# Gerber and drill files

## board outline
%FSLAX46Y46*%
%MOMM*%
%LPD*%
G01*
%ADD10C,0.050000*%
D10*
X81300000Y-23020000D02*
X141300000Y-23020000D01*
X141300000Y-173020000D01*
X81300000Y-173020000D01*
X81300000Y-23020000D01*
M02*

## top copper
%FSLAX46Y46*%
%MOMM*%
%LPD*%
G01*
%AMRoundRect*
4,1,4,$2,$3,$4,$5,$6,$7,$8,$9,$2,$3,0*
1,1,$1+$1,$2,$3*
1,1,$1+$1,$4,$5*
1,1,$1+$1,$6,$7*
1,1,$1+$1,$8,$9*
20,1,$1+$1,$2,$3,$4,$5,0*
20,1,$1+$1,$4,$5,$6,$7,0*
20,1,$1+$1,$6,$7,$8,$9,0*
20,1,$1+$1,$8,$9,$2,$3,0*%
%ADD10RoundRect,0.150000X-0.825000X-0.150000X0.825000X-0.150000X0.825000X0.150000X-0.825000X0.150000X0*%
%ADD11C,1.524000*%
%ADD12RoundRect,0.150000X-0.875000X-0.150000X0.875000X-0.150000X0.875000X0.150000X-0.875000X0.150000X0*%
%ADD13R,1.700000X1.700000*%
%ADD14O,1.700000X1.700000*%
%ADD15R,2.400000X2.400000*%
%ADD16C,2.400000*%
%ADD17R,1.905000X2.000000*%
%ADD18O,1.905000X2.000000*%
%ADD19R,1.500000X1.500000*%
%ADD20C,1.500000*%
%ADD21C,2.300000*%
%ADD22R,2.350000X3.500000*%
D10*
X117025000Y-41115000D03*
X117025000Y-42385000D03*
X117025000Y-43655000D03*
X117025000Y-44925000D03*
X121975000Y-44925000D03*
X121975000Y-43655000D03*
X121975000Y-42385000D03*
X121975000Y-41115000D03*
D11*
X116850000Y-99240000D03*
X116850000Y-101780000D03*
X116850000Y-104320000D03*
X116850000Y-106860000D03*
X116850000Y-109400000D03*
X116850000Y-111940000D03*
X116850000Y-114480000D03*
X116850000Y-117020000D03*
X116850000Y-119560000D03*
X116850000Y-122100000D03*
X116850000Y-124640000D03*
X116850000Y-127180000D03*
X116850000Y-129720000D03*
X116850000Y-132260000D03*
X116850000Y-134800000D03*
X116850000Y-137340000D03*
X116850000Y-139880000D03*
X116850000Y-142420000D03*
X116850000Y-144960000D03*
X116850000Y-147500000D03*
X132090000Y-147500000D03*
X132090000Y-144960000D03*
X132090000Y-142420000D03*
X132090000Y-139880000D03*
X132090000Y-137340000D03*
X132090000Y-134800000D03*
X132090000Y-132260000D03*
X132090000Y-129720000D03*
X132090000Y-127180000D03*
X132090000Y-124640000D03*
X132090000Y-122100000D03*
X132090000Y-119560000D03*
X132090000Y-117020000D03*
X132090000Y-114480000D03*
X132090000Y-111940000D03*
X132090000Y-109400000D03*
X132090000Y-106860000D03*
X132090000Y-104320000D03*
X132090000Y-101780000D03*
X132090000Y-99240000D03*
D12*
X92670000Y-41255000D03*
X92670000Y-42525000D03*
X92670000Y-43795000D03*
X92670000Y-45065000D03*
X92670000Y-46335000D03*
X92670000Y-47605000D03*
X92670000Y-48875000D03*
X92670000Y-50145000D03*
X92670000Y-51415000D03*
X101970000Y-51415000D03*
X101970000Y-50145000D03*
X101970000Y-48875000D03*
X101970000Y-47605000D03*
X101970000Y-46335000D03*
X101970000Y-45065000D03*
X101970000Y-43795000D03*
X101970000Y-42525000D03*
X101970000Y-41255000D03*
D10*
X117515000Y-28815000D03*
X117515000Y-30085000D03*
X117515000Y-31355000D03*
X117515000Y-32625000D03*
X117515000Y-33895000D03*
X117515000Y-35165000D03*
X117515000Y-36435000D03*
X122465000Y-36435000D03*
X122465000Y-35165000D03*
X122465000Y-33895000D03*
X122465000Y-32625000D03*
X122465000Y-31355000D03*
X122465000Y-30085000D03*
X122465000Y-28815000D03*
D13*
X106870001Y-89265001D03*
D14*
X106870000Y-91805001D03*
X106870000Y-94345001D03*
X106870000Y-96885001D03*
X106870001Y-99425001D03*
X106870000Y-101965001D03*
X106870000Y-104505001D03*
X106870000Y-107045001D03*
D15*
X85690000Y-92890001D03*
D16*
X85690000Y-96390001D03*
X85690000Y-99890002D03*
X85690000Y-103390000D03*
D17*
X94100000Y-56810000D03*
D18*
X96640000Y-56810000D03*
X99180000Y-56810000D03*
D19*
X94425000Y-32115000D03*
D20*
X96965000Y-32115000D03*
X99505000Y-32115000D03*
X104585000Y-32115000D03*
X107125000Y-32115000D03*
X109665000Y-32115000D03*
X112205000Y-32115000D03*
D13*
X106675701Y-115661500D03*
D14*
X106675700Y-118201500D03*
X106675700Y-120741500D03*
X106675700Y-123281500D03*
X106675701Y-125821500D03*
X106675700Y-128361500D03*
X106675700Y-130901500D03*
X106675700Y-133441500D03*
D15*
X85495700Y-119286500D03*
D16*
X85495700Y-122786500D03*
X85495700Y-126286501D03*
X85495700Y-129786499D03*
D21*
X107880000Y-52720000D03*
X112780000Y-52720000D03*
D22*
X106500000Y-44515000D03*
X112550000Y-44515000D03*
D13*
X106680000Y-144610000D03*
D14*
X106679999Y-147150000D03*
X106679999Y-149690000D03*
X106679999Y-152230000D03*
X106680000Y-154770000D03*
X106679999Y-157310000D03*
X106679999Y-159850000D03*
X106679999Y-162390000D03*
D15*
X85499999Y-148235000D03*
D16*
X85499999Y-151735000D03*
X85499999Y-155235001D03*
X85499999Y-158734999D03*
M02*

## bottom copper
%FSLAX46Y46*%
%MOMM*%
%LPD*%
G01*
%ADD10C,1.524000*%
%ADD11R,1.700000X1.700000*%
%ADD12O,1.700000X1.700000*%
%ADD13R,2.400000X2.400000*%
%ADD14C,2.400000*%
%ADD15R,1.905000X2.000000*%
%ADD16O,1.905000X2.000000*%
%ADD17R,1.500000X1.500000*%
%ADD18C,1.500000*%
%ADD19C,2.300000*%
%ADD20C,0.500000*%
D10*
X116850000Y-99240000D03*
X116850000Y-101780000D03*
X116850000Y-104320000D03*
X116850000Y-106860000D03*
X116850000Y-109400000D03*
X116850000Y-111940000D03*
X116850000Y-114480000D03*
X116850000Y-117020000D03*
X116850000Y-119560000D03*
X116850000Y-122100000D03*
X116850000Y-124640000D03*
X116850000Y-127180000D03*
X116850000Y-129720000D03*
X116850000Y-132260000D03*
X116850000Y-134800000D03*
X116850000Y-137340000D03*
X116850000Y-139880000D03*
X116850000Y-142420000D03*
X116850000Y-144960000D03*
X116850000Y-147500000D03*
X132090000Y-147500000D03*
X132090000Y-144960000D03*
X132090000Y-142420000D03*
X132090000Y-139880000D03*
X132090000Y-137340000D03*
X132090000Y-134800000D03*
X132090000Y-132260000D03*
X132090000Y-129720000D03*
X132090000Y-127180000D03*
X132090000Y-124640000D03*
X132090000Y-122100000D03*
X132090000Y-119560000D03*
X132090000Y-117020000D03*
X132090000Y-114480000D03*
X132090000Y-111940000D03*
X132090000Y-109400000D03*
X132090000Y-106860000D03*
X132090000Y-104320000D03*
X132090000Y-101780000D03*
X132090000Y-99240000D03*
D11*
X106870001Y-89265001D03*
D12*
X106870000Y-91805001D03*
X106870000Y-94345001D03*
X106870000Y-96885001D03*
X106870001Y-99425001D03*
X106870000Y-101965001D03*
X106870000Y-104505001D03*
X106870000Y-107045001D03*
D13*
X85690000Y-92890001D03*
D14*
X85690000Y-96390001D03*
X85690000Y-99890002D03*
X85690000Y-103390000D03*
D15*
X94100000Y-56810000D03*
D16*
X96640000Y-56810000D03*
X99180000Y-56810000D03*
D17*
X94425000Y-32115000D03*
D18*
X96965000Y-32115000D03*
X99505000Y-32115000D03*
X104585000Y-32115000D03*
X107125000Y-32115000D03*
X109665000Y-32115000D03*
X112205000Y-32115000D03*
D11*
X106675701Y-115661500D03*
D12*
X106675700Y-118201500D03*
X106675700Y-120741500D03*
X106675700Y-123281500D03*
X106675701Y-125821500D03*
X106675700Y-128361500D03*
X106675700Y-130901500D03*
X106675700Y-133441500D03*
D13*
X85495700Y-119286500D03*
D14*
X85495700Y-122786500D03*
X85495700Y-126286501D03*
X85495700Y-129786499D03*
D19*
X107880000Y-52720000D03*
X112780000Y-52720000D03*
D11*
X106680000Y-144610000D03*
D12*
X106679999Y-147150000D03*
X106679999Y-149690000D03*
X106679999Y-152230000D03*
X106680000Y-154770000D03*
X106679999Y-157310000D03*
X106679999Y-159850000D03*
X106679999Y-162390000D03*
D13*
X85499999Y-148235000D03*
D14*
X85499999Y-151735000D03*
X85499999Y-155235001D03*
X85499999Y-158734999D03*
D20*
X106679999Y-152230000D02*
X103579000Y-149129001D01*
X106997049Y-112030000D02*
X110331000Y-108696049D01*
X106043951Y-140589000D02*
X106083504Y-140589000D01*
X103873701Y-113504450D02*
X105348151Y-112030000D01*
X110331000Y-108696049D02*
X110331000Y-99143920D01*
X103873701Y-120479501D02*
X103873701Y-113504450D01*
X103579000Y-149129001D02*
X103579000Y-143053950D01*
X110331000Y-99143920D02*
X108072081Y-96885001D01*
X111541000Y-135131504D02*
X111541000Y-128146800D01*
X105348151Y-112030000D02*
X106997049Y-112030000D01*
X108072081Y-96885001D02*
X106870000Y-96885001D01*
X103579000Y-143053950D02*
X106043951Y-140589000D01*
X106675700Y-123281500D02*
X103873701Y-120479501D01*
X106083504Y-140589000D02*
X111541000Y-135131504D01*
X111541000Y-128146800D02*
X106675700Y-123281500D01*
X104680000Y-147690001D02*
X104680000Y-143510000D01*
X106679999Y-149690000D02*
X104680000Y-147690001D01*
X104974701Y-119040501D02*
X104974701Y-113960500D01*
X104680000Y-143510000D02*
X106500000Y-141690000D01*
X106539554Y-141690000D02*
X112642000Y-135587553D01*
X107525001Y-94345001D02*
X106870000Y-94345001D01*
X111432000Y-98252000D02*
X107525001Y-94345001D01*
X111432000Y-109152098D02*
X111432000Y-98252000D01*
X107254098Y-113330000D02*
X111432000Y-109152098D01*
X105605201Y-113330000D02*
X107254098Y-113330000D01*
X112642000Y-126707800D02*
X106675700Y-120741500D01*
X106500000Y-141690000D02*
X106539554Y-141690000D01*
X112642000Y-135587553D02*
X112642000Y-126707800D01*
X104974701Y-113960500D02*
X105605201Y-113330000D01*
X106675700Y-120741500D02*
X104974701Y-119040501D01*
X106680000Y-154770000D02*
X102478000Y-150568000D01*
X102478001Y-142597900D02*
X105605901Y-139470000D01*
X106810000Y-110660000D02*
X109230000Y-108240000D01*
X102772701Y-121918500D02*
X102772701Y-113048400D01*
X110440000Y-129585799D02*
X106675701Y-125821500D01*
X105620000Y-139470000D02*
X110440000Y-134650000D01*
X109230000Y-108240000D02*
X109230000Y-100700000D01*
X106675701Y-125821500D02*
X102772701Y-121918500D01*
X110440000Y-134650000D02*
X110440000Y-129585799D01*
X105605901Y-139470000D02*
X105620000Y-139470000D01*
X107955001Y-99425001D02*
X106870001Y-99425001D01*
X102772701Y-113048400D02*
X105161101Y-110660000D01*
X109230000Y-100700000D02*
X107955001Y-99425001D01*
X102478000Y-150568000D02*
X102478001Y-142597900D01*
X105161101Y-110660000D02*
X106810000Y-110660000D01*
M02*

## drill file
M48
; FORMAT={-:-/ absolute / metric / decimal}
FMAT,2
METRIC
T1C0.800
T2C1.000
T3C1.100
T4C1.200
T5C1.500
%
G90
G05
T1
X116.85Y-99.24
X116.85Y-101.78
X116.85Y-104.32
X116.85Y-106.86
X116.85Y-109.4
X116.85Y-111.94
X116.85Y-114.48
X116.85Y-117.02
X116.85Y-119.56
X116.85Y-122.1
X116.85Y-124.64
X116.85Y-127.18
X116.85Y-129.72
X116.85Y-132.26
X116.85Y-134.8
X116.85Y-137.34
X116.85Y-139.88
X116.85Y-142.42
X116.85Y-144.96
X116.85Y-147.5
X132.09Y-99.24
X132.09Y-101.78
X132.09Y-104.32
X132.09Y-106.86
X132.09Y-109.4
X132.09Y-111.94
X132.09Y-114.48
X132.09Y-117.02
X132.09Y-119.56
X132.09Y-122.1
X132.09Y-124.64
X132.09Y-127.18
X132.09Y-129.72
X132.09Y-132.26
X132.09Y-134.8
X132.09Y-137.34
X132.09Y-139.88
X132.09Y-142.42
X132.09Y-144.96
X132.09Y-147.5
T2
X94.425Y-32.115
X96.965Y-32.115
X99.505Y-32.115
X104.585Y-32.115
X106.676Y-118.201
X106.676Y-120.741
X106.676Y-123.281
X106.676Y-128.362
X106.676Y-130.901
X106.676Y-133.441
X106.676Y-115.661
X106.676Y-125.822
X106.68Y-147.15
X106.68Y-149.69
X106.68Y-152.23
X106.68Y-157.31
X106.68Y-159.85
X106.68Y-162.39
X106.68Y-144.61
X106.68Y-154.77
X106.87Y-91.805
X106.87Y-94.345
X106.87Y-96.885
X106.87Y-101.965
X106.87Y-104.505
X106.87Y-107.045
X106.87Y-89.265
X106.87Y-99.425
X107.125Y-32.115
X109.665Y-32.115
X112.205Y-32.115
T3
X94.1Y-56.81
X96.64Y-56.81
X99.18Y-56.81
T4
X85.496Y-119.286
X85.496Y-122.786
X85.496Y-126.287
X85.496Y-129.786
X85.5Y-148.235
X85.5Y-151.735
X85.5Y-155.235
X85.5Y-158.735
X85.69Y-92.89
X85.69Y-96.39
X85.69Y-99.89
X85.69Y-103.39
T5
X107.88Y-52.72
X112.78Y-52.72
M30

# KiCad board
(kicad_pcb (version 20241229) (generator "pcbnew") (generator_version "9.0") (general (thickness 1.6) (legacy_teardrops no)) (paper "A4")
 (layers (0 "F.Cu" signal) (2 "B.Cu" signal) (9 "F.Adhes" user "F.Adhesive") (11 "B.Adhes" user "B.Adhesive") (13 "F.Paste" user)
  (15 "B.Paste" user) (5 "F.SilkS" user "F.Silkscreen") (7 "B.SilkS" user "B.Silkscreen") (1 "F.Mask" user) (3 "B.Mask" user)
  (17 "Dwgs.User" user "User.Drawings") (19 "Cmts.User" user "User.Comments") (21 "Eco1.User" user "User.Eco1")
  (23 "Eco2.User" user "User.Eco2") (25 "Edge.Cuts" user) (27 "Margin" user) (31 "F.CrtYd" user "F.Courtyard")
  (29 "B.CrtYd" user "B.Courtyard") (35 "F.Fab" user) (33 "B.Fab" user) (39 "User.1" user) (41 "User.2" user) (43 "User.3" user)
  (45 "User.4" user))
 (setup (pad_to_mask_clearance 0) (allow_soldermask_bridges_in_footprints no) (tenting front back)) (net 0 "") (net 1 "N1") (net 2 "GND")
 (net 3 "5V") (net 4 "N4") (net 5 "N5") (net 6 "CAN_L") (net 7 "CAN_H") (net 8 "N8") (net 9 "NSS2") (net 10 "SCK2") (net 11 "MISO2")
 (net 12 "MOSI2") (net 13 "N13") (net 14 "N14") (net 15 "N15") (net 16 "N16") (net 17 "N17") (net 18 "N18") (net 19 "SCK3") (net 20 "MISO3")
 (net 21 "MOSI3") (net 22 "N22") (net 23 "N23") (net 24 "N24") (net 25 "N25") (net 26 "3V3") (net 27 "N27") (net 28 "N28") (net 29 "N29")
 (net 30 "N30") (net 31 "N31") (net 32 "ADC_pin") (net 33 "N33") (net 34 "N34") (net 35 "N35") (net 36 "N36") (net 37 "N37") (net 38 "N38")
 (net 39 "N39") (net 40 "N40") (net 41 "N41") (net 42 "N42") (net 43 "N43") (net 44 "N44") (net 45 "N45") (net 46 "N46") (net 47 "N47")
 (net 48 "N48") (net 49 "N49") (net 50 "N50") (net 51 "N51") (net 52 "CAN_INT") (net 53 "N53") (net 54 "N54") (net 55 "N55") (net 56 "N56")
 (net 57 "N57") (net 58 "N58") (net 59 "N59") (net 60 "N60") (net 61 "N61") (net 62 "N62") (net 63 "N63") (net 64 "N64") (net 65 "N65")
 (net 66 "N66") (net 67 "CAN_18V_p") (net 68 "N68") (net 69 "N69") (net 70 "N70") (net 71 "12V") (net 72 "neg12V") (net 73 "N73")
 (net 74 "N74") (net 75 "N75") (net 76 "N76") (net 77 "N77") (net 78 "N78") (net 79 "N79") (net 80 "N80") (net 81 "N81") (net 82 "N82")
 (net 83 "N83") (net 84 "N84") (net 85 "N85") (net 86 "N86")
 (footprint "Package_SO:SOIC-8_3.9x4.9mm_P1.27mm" (layer "F.Cu") (at 119.5 43.02)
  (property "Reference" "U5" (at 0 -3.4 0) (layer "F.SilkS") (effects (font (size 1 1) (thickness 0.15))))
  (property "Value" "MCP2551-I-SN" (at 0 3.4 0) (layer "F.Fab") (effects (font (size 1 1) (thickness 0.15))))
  (pad "1" smd roundrect (at -2.475 -1.905) (size 1.95 0.6) (layers "F.Cu" "F.Mask" "F.Paste") (roundrect_rratio 0.25) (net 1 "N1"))
  (pad "2" smd roundrect (at -2.475 -0.635) (size 1.95 0.6) (layers "F.Cu" "F.Mask" "F.Paste") (roundrect_rratio 0.25) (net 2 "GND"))
  (pad "3" smd roundrect (at -2.475 0.635) (size 1.95 0.6) (layers "F.Cu" "F.Mask" "F.Paste") (roundrect_rratio 0.25) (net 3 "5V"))
  (pad "4" smd roundrect (at -2.475 1.905) (size 1.95 0.6) (layers "F.Cu" "F.Mask" "F.Paste") (roundrect_rratio 0.25) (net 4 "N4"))
  (pad "5" smd roundrect (at 2.475 1.905) (size 1.95 0.6) (layers "F.Cu" "F.Mask" "F.Paste") (roundrect_rratio 0.25) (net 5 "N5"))
  (pad "6" smd roundrect (at 2.475 0.635) (size 1.95 0.6) (layers "F.Cu" "F.Mask" "F.Paste") (roundrect_rratio 0.25) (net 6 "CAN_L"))
  (pad "7" smd roundrect (at 2.475 -0.635) (size 1.95 0.6) (layers "F.Cu" "F.Mask" "F.Paste") (roundrect_rratio 0.25) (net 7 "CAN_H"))
  (pad "8" smd roundrect (at 2.475 -1.905) (size 1.95 0.6) (layers "F.Cu" "F.Mask" "F.Paste") (roundrect_rratio 0.25) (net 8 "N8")))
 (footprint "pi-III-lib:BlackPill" (layer "F.Cu") (at 124.47 120.83)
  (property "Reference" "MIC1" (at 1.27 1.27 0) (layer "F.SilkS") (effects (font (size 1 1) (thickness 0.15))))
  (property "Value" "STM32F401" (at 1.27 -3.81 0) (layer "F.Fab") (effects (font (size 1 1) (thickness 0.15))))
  (pad "1" thru_hole circle (at -7.62 -21.59) (size 1.524 1.524) (drill 0.8) (layers "*.Cu" "*.Mask") (remove_unused_layers no)
   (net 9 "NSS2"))
  (pad "2" thru_hole circle (at -7.62 -19.05) (size 1.524 1.524) (drill 0.8) (layers "*.Cu" "*.Mask") (remove_unused_layers no)
   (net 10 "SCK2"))
  (pad "3" thru_hole circle (at -7.62 -16.51) (size 1.524 1.524) (drill 0.8) (layers "*.Cu" "*.Mask") (remove_unused_layers no)
   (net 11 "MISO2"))
  (pad "4" thru_hole circle (at -7.62 -13.97) (size 1.524 1.524) (drill 0.8) (layers "*.Cu" "*.Mask") (remove_unused_layers no)
   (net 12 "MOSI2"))
  (pad "5" thru_hole circle (at -7.62 -11.43) (size 1.524 1.524) (drill 0.8) (layers "*.Cu" "*.Mask") (remove_unused_layers no)
   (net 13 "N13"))
  (pad "6" thru_hole circle (at -7.62 -8.89) (size 1.524 1.524) (drill 0.8) (layers "*.Cu" "*.Mask") (remove_unused_layers no)
   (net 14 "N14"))
  (pad "7" thru_hole circle (at -7.62 -6.35) (size 1.524 1.524) (drill 0.8) (layers "*.Cu" "*.Mask") (remove_unused_layers no)
   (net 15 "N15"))
  (pad "8" thru_hole circle (at -7.62 -3.81) (size 1.524 1.524) (drill 0.8) (layers "*.Cu" "*.Mask") (remove_unused_layers no)
   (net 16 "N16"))
  (pad "9" thru_hole circle (at -7.62 -1.27) (size 1.524 1.524) (drill 0.8) (layers "*.Cu" "*.Mask") (remove_unused_layers no)
   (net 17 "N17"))
  (pad "10" thru_hole circle (at -7.62 1.27) (size 1.524 1.524) (drill 0.8) (layers "*.Cu" "*.Mask") (remove_unused_layers no)
   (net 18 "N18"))
  (pad "11" thru_hole circle (at -7.62 3.81) (size 1.524 1.524) (drill 0.8) (layers "*.Cu" "*.Mask") (remove_unused_layers no)
   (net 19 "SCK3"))
  (pad "12" thru_hole circle (at -7.62 6.35) (size 1.524 1.524) (drill 0.8) (layers "*.Cu" "*.Mask") (remove_unused_layers no)
   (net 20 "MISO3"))
  (pad "13" thru_hole circle (at -7.62 8.89) (size 1.524 1.524) (drill 0.8) (layers "*.Cu" "*.Mask") (remove_unused_layers no)
   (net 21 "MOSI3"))
  (pad "14" thru_hole circle (at -7.62 11.43) (size 1.524 1.524) (drill 0.8) (layers "*.Cu" "*.Mask") (remove_unused_layers no)
   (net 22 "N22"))
  (pad "15" thru_hole circle (at -7.62 13.97) (size 1.524 1.524) (drill 0.8) (layers "*.Cu" "*.Mask") (remove_unused_layers no)
   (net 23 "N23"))
  (pad "16" thru_hole circle (at -7.62 16.51) (size 1.524 1.524) (drill 0.8) (layers "*.Cu" "*.Mask") (remove_unused_layers no)
   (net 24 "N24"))
  (pad "17" thru_hole circle (at -7.62 19.05) (size 1.524 1.524) (drill 0.8) (layers "*.Cu" "*.Mask") (remove_unused_layers no)
   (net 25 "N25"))
  (pad "18" thru_hole circle (at -7.62 21.59) (size 1.524 1.524) (drill 0.8) (layers "*.Cu" "*.Mask") (remove_unused_layers no) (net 3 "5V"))
  (pad "19" thru_hole circle (at -7.62 24.13) (size 1.524 1.524) (drill 0.8) (layers "*.Cu" "*.Mask") (remove_unused_layers no)
   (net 2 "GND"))
  (pad "20" thru_hole circle (at -7.62 26.67) (size 1.524 1.524) (drill 0.8) (layers "*.Cu" "*.Mask") (remove_unused_layers no)
   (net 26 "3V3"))
  (pad "21" thru_hole circle (at 7.62 26.67) (size 1.524 1.524) (drill 0.8) (layers "*.Cu" "*.Mask") (remove_unused_layers no)
   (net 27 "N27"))
  (pad "22" thru_hole circle (at 7.62 24.13) (size 1.524 1.524) (drill 0.8) (layers "*.Cu" "*.Mask") (remove_unused_layers no)
   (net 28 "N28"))
  (pad "23" thru_hole circle (at 7.62 21.59) (size 1.524 1.524) (drill 0.8) (layers "*.Cu" "*.Mask") (remove_unused_layers no)
   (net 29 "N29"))
  (pad "24" thru_hole circle (at 7.62 19.05) (size 1.524 1.524) (drill 0.8) (layers "*.Cu" "*.Mask") (remove_unused_layers no)
   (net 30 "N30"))
  (pad "25" thru_hole circle (at 7.62 16.51) (size 1.524 1.524) (drill 0.8) (layers "*.Cu" "*.Mask") (remove_unused_layers no)
   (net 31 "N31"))
  (pad "26" thru_hole circle (at 7.62 13.97) (size 1.524 1.524) (drill 0.8) (layers "*.Cu" "*.Mask") (remove_unused_layers no)
   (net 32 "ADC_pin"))
  (pad "27" thru_hole circle (at 7.62 11.43) (size 1.524 1.524) (drill 0.8) (layers "*.Cu" "*.Mask") (remove_unused_layers no)
   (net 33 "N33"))
  (pad "28" thru_hole circle (at 7.62 8.89) (size 1.524 1.524) (drill 0.8) (layers "*.Cu" "*.Mask") (remove_unused_layers no) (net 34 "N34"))
  (pad "29" thru_hole circle (at 7.62 6.35) (size 1.524 1.524) (drill 0.8) (layers "*.Cu" "*.Mask") (remove_unused_layers no) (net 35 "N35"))
  (pad "30" thru_hole circle (at 7.62 3.81) (size 1.524 1.524) (drill 0.8) (layers "*.Cu" "*.Mask") (remove_unused_layers no) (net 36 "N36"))
  (pad "31" thru_hole circle (at 7.62 1.27) (size 1.524 1.524) (drill 0.8) (layers "*.Cu" "*.Mask") (remove_unused_layers no) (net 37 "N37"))
  (pad "32" thru_hole circle (at 7.62 -1.27) (size 1.524 1.524) (drill 0.8) (layers "*.Cu" "*.Mask") (remove_unused_layers no)
   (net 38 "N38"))
  (pad "33" thru_hole circle (at 7.62 -3.81) (size 1.524 1.524) (drill 0.8) (layers "*.Cu" "*.Mask") (remove_unused_layers no)
   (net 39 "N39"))
  (pad "34" thru_hole circle (at 7.62 -6.35) (size 1.524 1.524) (drill 0.8) (layers "*.Cu" "*.Mask") (remove_unused_layers no)
   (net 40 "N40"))
  (pad "35" thru_hole circle (at 7.62 -8.89) (size 1.524 1.524) (drill 0.8) (layers "*.Cu" "*.Mask") (remove_unused_layers no)
   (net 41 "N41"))
  (pad "36" thru_hole circle (at 7.62 -11.43) (size 1.524 1.524) (drill 0.8) (layers "*.Cu" "*.Mask") (remove_unused_layers no)
   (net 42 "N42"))
  (pad "37" thru_hole circle (at 7.62 -13.97) (size 1.524 1.524) (drill 0.8) (layers "*.Cu" "*.Mask") (remove_unused_layers no)
   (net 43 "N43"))
  (pad "38" thru_hole circle (at 7.62 -16.51) (size 1.524 1.524) (drill 0.8) (layers "*.Cu" "*.Mask") (remove_unused_layers no)
   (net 26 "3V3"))
  (pad "39" thru_hole circle (at 7.62 -19.05) (size 1.524 1.524) (drill 0.8) (layers "*.Cu" "*.Mask") (remove_unused_layers no)
   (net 2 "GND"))
  (pad "40" thru_hole circle (at 7.62 -21.59) (size 1.524 1.524) (drill 0.8) (layers "*.Cu" "*.Mask") (remove_unused_layers no) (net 3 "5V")))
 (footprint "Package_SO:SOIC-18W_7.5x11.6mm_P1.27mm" (layer "F.Cu") (at 97.32 46.335)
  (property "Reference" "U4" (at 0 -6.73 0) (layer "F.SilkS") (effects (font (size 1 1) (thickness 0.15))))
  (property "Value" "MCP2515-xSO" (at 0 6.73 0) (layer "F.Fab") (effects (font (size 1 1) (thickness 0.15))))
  (pad "1" smd roundrect (at -4.65 -5.08) (size 2.05 0.6) (layers "F.Cu" "F.Mask" "F.Paste") (roundrect_rratio 0.25) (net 1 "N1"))
  (pad "2" smd roundrect (at -4.65 -3.81) (size 2.05 0.6) (layers "F.Cu" "F.Mask" "F.Paste") (roundrect_rratio 0.25) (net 4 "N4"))
  (pad "3" smd roundrect (at -4.65 -2.54) (size 2.05 0.6) (layers "F.Cu" "F.Mask" "F.Paste") (roundrect_rratio 0.25) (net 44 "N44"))
  (pad "4" smd roundrect (at -4.65 -1.27) (size 2.05 0.6) (layers "F.Cu" "F.Mask" "F.Paste") (roundrect_rratio 0.25) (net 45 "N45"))
  (pad "5" smd roundrect (at -4.65 0) (size 2.05 0.6) (layers "F.Cu" "F.Mask" "F.Paste") (roundrect_rratio 0.25) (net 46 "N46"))
  (pad "6" smd roundrect (at -4.65 1.27) (size 2.05 0.6) (layers "F.Cu" "F.Mask" "F.Paste") (roundrect_rratio 0.25) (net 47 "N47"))
  (pad "7" smd roundrect (at -4.65 2.54) (size 2.05 0.6) (layers "F.Cu" "F.Mask" "F.Paste") (roundrect_rratio 0.25) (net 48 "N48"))
  (pad "8" smd roundrect (at -4.65 3.81) (size 2.05 0.6) (layers "F.Cu" "F.Mask" "F.Paste") (roundrect_rratio 0.25) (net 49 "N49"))
  (pad "9" smd roundrect (at -4.65 5.08) (size 2.05 0.6) (layers "F.Cu" "F.Mask" "F.Paste") (roundrect_rratio 0.25) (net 2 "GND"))
  (pad "10" smd roundrect (at 4.65 5.08) (size 2.05 0.6) (layers "F.Cu" "F.Mask" "F.Paste") (roundrect_rratio 0.25) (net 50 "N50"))
  (pad "11" smd roundrect (at 4.65 3.81) (size 2.05 0.6) (layers "F.Cu" "F.Mask" "F.Paste") (roundrect_rratio 0.25) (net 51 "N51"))
  (pad "12" smd roundrect (at 4.65 2.54) (size 2.05 0.6) (layers "F.Cu" "F.Mask" "F.Paste") (roundrect_rratio 0.25) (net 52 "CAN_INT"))
  (pad "13" smd roundrect (at 4.65 1.27) (size 2.05 0.6) (layers "F.Cu" "F.Mask" "F.Paste") (roundrect_rratio 0.25) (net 10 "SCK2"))
  (pad "14" smd roundrect (at 4.65 0) (size 2.05 0.6) (layers "F.Cu" "F.Mask" "F.Paste") (roundrect_rratio 0.25) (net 12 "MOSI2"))
  (pad "15" smd roundrect (at 4.65 -1.27) (size 2.05 0.6) (layers "F.Cu" "F.Mask" "F.Paste") (roundrect_rratio 0.25) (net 11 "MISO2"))
  (pad "16" smd roundrect (at 4.65 -2.54) (size 2.05 0.6) (layers "F.Cu" "F.Mask" "F.Paste") (roundrect_rratio 0.25) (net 9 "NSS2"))
  (pad "17" smd roundrect (at 4.65 -3.81) (size 2.05 0.6) (layers "F.Cu" "F.Mask" "F.Paste") (roundrect_rratio 0.25) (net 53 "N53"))
  (pad "18" smd roundrect (at 4.65 -5.08) (size 2.05 0.6) (layers "F.Cu" "F.Mask" "F.Paste") (roundrect_rratio 0.25) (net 26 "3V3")))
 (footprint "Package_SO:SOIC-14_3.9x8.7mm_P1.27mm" (layer "F.Cu") (at 119.99 32.625)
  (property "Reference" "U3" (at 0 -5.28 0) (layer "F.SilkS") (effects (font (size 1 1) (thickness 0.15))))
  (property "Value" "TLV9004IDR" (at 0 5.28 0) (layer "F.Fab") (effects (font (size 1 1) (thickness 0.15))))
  (pad "1" smd roundrect (at -2.475 -3.81) (size 1.95 0.6) (layers "F.Cu" "F.Mask" "F.Paste") (roundrect_rratio 0.25) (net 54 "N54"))
  (pad "2" smd roundrect (at -2.475 -2.54) (size 1.95 0.6) (layers "F.Cu" "F.Mask" "F.Paste") (roundrect_rratio 0.25) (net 54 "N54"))
  (pad "3" smd roundrect (at -2.475 -1.27) (size 1.95 0.6) (layers "F.Cu" "F.Mask" "F.Paste") (roundrect_rratio 0.25) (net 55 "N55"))
  (pad "4" smd roundrect (at -2.475 0) (size 1.95 0.6) (layers "F.Cu" "F.Mask" "F.Paste") (roundrect_rratio 0.25) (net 26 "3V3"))
  (pad "5" smd roundrect (at -2.475 1.27) (size 1.95 0.6) (layers "F.Cu" "F.Mask" "F.Paste") (roundrect_rratio 0.25))
  (pad "6" smd roundrect (at -2.475 2.54) (size 1.95 0.6) (layers "F.Cu" "F.Mask" "F.Paste") (roundrect_rratio 0.25))
  (pad "7" smd roundrect (at -2.475 3.81) (size 1.95 0.6) (layers "F.Cu" "F.Mask" "F.Paste") (roundrect_rratio 0.25))
  (pad "8" smd roundrect (at 2.475 3.81) (size 1.95 0.6) (layers "F.Cu" "F.Mask" "F.Paste") (roundrect_rratio 0.25) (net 32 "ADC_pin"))
  (pad "9" smd roundrect (at 2.475 2.54) (size 1.95 0.6) (layers "F.Cu" "F.Mask" "F.Paste") (roundrect_rratio 0.25) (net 32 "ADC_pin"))
  (pad "10" smd roundrect (at 2.475 1.27) (size 1.95 0.6) (layers "F.Cu" "F.Mask" "F.Paste") (roundrect_rratio 0.25) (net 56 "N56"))
  (pad "11" smd roundrect (at 2.475 0) (size 1.95 0.6) (layers "F.Cu" "F.Mask" "F.Paste") (roundrect_rratio 0.25) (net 2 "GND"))
  (pad "12" smd roundrect (at 2.475 -1.27) (size 1.95 0.6) (layers "F.Cu" "F.Mask" "F.Paste") (roundrect_rratio 0.25) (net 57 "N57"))
  (pad "13" smd roundrect (at 2.475 -2.54) (size 1.95 0.6) (layers "F.Cu" "F.Mask" "F.Paste") (roundrect_rratio 0.25) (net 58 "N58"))
  (pad "14" smd roundrect (at 2.475 -3.81) (size 1.95 0.6) (layers "F.Cu" "F.Mask" "F.Paste") (roundrect_rratio 0.25) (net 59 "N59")))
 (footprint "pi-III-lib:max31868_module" (layer "F.Cu") (at 73.31 101.059501 90)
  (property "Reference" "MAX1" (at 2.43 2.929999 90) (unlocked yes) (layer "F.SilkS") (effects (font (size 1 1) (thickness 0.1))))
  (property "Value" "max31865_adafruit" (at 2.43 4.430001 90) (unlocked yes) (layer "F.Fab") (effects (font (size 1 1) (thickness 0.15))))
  (pad "1" thru_hole rect (at 11.7945 33.560001 180) (size 1.7 1.7) (drill 1) (layers "*.Cu" "*.Mask") (remove_unused_layers no)
   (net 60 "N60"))
  (pad "2" thru_hole oval (at 9.2545 33.56 180) (size 1.7 1.7) (drill 1) (layers "*.Cu" "*.Mask") (remove_unused_layers no) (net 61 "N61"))
  (pad "3" thru_hole oval (at 6.7145 33.56 180) (size 1.7 1.7) (drill 1) (layers "*.Cu" "*.Mask") (remove_unused_layers no) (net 21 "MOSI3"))
  (pad "4" thru_hole oval (at 4.1745 33.56 180) (size 1.7 1.7) (drill 1) (layers "*.Cu" "*.Mask") (remove_unused_layers no) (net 20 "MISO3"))
  (pad "5" thru_hole oval (at 1.6345 33.560001 180) (size 1.7 1.7) (drill 1) (layers "*.Cu" "*.Mask") (remove_unused_layers no)
   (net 19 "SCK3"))
  (pad "6" thru_hole oval (at -0.9055 33.56 180) (size 1.7 1.7) (drill 1) (layers "*.Cu" "*.Mask") (remove_unused_layers no) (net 26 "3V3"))
  (pad "7" thru_hole oval (at -3.4455 33.56 180) (size 1.7 1.7) (drill 1) (layers "*.Cu" "*.Mask") (remove_unused_layers no) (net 2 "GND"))
  (pad "8" thru_hole oval (at -5.9855 33.56 180) (size 1.7 1.7) (drill 1) (layers "*.Cu" "*.Mask") (remove_unused_layers no) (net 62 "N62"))
  (pad "9" thru_hole rect (at 8.1695 12.38 270) (size 2.4 2.4) (drill 1.2) (layers "*.Cu" "*.Mask") (remove_unused_layers no) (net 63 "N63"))
  (pad "10" thru_hole circle (at 4.6695 12.38 270) (size 2.4 2.4) (drill 1.2) (layers "*.Cu" "*.Mask") (remove_unused_layers no)
   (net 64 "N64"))
  (pad "11" thru_hole circle (at 1.169499 12.38 270) (size 2.4 2.4) (drill 1.2) (layers "*.Cu" "*.Mask") (remove_unused_layers no)
   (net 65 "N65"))
  (pad "12" thru_hole circle (at -2.330499 12.38 270) (size 2.4 2.4) (drill 1.2) (layers "*.Cu" "*.Mask") (remove_unused_layers no)
   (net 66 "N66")))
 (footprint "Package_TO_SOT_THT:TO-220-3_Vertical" (layer "F.Cu") (at 94.1 56.81)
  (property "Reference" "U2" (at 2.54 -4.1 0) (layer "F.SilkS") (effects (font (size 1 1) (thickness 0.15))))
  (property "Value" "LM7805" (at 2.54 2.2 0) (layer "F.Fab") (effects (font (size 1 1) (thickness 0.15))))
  (pad "1" thru_hole rect (at 0 0) (size 1.905 2) (drill 1.1) (layers "*.Cu" "*.Mask") (remove_unused_layers no) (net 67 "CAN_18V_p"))
  (pad "2" thru_hole oval (at 2.54 0) (size 1.905 2) (drill 1.1) (layers "*.Cu" "*.Mask") (remove_unused_layers no) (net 2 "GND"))
  (pad "3" thru_hole oval (at 5.08 0) (size 1.905 2) (drill 1.1) (layers "*.Cu" "*.Mask") (remove_unused_layers no) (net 3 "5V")))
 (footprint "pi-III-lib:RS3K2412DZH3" (layer "F.Cu") (at 94.425 32.115)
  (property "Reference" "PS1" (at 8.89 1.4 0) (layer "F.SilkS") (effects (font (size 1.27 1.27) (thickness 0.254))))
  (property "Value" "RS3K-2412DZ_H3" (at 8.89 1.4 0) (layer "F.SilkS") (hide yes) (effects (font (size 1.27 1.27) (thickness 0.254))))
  (pad "1" thru_hole rect (at 0 0) (size 1.5 1.5) (drill 1) (layers "*.Cu" "*.Mask") (remove_unused_layers no) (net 2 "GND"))
  (pad "2" thru_hole circle (at 2.54 0) (size 1.5 1.5) (drill 1) (layers "*.Cu" "*.Mask") (remove_unused_layers no) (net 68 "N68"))
  (pad "3" thru_hole circle (at 5.08 0) (size 1.5 1.5) (drill 1) (layers "*.Cu" "*.Mask") (remove_unused_layers no) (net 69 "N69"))
  (pad "5" thru_hole circle (at 10.16 0) (size 1.5 1.5) (drill 1) (layers "*.Cu" "*.Mask") (remove_unused_layers no) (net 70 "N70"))
  (pad "6" thru_hole circle (at 12.7 0) (size 1.5 1.5) (drill 1) (layers "*.Cu" "*.Mask") (remove_unused_layers no) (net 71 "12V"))
  (pad "7" thru_hole circle (at 15.24 0) (size 1.5 1.5) (drill 1) (layers "*.Cu" "*.Mask") (remove_unused_layers no) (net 2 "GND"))
  (pad "8" thru_hole circle (at 17.78 0) (size 1.5 1.5) (drill 1) (layers "*.Cu" "*.Mask") (remove_unused_layers no) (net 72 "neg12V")))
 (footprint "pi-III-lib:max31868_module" (layer "F.Cu") (at 73.1157 127.456 90)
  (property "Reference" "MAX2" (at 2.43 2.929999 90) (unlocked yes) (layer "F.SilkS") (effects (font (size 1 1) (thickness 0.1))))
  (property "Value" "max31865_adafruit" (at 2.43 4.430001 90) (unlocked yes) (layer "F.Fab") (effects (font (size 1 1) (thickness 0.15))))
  (pad "1" thru_hole rect (at 11.7945 33.560001 180) (size 1.7 1.7) (drill 1) (layers "*.Cu" "*.Mask") (remove_unused_layers no)
   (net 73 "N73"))
  (pad "2" thru_hole oval (at 9.2545 33.56 180) (size 1.7 1.7) (drill 1) (layers "*.Cu" "*.Mask") (remove_unused_layers no) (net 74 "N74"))
  (pad "3" thru_hole oval (at 6.7145 33.56 180) (size 1.7 1.7) (drill 1) (layers "*.Cu" "*.Mask") (remove_unused_layers no) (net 21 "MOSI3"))
  (pad "4" thru_hole oval (at 4.1745 33.56 180) (size 1.7 1.7) (drill 1) (layers "*.Cu" "*.Mask") (remove_unused_layers no) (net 20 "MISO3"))
  (pad "5" thru_hole oval (at 1.6345 33.560001 180) (size 1.7 1.7) (drill 1) (layers "*.Cu" "*.Mask") (remove_unused_layers no)
   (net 19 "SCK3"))
  (pad "6" thru_hole oval (at -0.9055 33.56 180) (size 1.7 1.7) (drill 1) (layers "*.Cu" "*.Mask") (remove_unused_layers no) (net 26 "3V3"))
  (pad "7" thru_hole oval (at -3.4455 33.56 180) (size 1.7 1.7) (drill 1) (layers "*.Cu" "*.Mask") (remove_unused_layers no) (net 2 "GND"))
  (pad "8" thru_hole oval (at -5.9855 33.56 180) (size 1.7 1.7) (drill 1) (layers "*.Cu" "*.Mask") (remove_unused_layers no) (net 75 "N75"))
  (pad "9" thru_hole rect (at 8.1695 12.38 270) (size 2.4 2.4) (drill 1.2) (layers "*.Cu" "*.Mask") (remove_unused_layers no) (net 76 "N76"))
  (pad "10" thru_hole circle (at 4.6695 12.38 270) (size 2.4 2.4) (drill 1.2) (layers "*.Cu" "*.Mask") (remove_unused_layers no)
   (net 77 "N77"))
  (pad "11" thru_hole circle (at 1.169499 12.38 270) (size 2.4 2.4) (drill 1.2) (layers "*.Cu" "*.Mask") (remove_unused_layers no)
   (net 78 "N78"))
  (pad "12" thru_hole circle (at -2.330499 12.38 270) (size 2.4 2.4) (drill 1.2) (layers "*.Cu" "*.Mask") (remove_unused_layers no)
   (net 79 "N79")))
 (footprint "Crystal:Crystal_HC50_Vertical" (layer "F.Cu") (at 107.88 52.72)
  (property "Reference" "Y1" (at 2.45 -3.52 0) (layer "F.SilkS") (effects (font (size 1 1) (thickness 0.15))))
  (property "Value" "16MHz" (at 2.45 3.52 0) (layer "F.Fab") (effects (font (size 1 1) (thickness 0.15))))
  (pad "1" thru_hole circle (at 0 0) (size 2.3 2.3) (drill 1.5) (layers "*.Cu" "*.Mask") (remove_unused_layers no) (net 49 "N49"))
  (pad "2" thru_hole circle (at 4.9 0) (size 2.3 2.3) (drill 1.5) (layers "*.Cu" "*.Mask") (remove_unused_layers no) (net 48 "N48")))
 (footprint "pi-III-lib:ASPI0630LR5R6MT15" (layer "F.Cu") (at 109.525 44.515)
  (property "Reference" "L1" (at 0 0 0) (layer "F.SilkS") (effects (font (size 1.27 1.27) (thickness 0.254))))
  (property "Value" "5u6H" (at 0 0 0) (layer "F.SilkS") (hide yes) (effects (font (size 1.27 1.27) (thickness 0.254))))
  (pad "1" smd rect (at -3.025 0) (size 2.35 3.5) (layers "F.Cu" "F.Mask" "F.Paste") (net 67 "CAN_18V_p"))
  (pad "2" smd rect (at 3.025 0) (size 2.35 3.5) (layers "F.Cu" "F.Mask" "F.Paste") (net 68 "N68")))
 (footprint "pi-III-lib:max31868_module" (layer "F.Cu") (at 73.119999 156.4045 90)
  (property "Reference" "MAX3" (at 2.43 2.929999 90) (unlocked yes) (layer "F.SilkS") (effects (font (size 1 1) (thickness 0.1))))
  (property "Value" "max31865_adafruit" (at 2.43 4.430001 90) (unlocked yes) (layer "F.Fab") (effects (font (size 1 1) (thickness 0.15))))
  (pad "1" thru_hole rect (at 11.7945 33.560001 180) (size 1.7 1.7) (drill 1) (layers "*.Cu" "*.Mask") (remove_unused_layers no)
   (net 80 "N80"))
  (pad "2" thru_hole oval (at 9.2545 33.56 180) (size 1.7 1.7) (drill 1) (layers "*.Cu" "*.Mask") (remove_unused_layers no) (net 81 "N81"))
  (pad "3" thru_hole oval (at 6.7145 33.56 180) (size 1.7 1.7) (drill 1) (layers "*.Cu" "*.Mask") (remove_unused_layers no) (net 21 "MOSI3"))
  (pad "4" thru_hole oval (at 4.1745 33.56 180) (size 1.7 1.7) (drill 1) (layers "*.Cu" "*.Mask") (remove_unused_layers no) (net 20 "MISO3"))
  (pad "5" thru_hole oval (at 1.6345 33.560001 180) (size 1.7 1.7) (drill 1) (layers "*.Cu" "*.Mask") (remove_unused_layers no)
   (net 19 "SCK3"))
  (pad "6" thru_hole oval (at -0.9055 33.56 180) (size 1.7 1.7) (drill 1) (layers "*.Cu" "*.Mask") (remove_unused_layers no) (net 26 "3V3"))
  (pad "7" thru_hole oval (at -3.4455 33.56 180) (size 1.7 1.7) (drill 1) (layers "*.Cu" "*.Mask") (remove_unused_layers no) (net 2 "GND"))
  (pad "8" thru_hole oval (at -5.9855 33.56 180) (size 1.7 1.7) (drill 1) (layers "*.Cu" "*.Mask") (remove_unused_layers no) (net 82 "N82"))
  (pad "9" thru_hole rect (at 8.1695 12.38 270) (size 2.4 2.4) (drill 1.2) (layers "*.Cu" "*.Mask") (remove_unused_layers no) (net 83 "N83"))
  (pad "10" thru_hole circle (at 4.6695 12.38 270) (size 2.4 2.4) (drill 1.2) (layers "*.Cu" "*.Mask") (remove_unused_layers no)
   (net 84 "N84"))
  (pad "11" thru_hole circle (at 1.169499 12.38 270) (size 2.4 2.4) (drill 1.2) (layers "*.Cu" "*.Mask") (remove_unused_layers no)
   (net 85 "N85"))
  (pad "12" thru_hole circle (at -2.330499 12.38 270) (size 2.4 2.4) (drill 1.2) (layers "*.Cu" "*.Mask") (remove_unused_layers no)
   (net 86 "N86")))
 (gr_rect (start 81.3 23.02) (end 141.3 173.02) (stroke (width 0.05) (type solid)) (fill no) (layer "Edge.Cuts"))
 (segment (start 106.679999 152.23) (end 103.579 149.129001) (width 0.5) (layer "B.Cu") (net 20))
 (segment (start 106.997049 112.03) (end 110.331 108.696049) (width 0.5) (layer "B.Cu") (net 20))
 (segment (start 106.043951 140.589) (end 106.083504 140.589) (width 0.5) (layer "B.Cu") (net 20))
 (segment (start 103.873701 113.50445) (end 105.348151 112.03) (width 0.5) (layer "B.Cu") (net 20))
 (segment (start 110.331 108.696049) (end 110.331 99.14392) (width 0.5) (layer "B.Cu") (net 20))
 (segment (start 103.873701 120.479501) (end 103.873701 113.50445) (width 0.5) (layer "B.Cu") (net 20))
 (segment (start 103.579 149.129001) (end 103.579 143.05395) (width 0.5) (layer "B.Cu") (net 20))
 (segment (start 110.331 99.14392) (end 108.072081 96.885001) (width 0.5) (layer "B.Cu") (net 20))
 (segment (start 111.541 135.131504) (end 111.541 128.1468) (width 0.5) (layer "B.Cu") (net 20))
 (segment (start 105.348151 112.03) (end 106.997049 112.03) (width 0.5) (layer "B.Cu") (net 20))
 (segment (start 108.072081 96.885001) (end 106.87 96.885001) (width 0.5) (layer "B.Cu") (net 20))
 (segment (start 103.579 143.05395) (end 106.043951 140.589) (width 0.5) (layer "B.Cu") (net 20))
 (segment (start 106.6757 123.2815) (end 103.873701 120.479501) (width 0.5) (layer "B.Cu") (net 20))
 (segment (start 106.083504 140.589) (end 111.541 135.131504) (width 0.5) (layer "B.Cu") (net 20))
 (segment (start 111.541 128.1468) (end 106.6757 123.2815) (width 0.5) (layer "B.Cu") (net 20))
 (segment (start 104.68 147.690001) (end 104.68 143.51) (width 0.5) (layer "B.Cu") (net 21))
 (segment (start 106.679999 149.69) (end 104.68 147.690001) (width 0.5) (layer "B.Cu") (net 21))
 (segment (start 104.974701 119.040501) (end 104.974701 113.9605) (width 0.5) (layer "B.Cu") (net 21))
 (segment (start 104.68 143.51) (end 106.5 141.69) (width 0.5) (layer "B.Cu") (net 21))
 (segment (start 106.539554 141.69) (end 112.642 135.587553) (width 0.5) (layer "B.Cu") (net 21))
 (segment (start 107.525001 94.345001) (end 106.87 94.345001) (width 0.5) (layer "B.Cu") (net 21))
 (segment (start 111.432 98.252) (end 107.525001 94.345001) (width 0.5) (layer "B.Cu") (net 21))
 (segment (start 111.432 109.152098) (end 111.432 98.252) (width 0.5) (layer "B.Cu") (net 21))
 (segment (start 107.254098 113.33) (end 111.432 109.152098) (width 0.5) (layer "B.Cu") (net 21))
 (segment (start 105.605201 113.33) (end 107.254098 113.33) (width 0.5) (layer "B.Cu") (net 21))
 (segment (start 112.642 126.7078) (end 106.6757 120.7415) (width 0.5) (layer "B.Cu") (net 21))
 (segment (start 106.5 141.69) (end 106.539554 141.69) (width 0.5) (layer "B.Cu") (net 21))
 (segment (start 112.642 135.587553) (end 112.642 126.7078) (width 0.5) (layer "B.Cu") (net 21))
 (segment (start 104.974701 113.9605) (end 105.605201 113.33) (width 0.5) (layer "B.Cu") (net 21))
 (segment (start 106.6757 120.7415) (end 104.974701 119.040501) (width 0.5) (layer "B.Cu") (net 21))
 (segment (start 106.68 154.77) (end 102.478 150.568) (width 0.5) (layer "B.Cu") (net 19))
 (segment (start 102.478001 142.5979) (end 105.605901 139.47) (width 0.5) (layer "B.Cu") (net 19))
 (segment (start 106.81 110.66) (end 109.23 108.24) (width 0.5) (layer "B.Cu") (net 19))
 (segment (start 102.772701 121.9185) (end 102.772701 113.0484) (width 0.5) (layer "B.Cu") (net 19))
 (segment (start 110.44 129.585799) (end 106.675701 125.8215) (width 0.5) (layer "B.Cu") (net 19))
 (segment (start 105.62 139.47) (end 110.44 134.65) (width 0.5) (layer "B.Cu") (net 19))
 (segment (start 109.23 108.24) (end 109.23 100.7) (width 0.5) (layer "B.Cu") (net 19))
 (segment (start 106.675701 125.8215) (end 102.772701 121.9185) (width 0.5) (layer "B.Cu") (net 19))
 (segment (start 110.44 134.65) (end 110.44 129.585799) (width 0.5) (layer "B.Cu") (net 19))
 (segment (start 105.605901 139.47) (end 105.62 139.47) (width 0.5) (layer "B.Cu") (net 19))
 (segment (start 107.955001 99.425001) (end 106.870001 99.425001) (width 0.5) (layer "B.Cu") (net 19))
 (segment (start 102.772701 113.0484) (end 105.161101 110.66) (width 0.5) (layer "B.Cu") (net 19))
 (segment (start 109.23 100.7) (end 107.955001 99.425001) (width 0.5) (layer "B.Cu") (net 19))
 (segment (start 102.478 150.568) (end 102.478001 142.5979) (width 0.5) (layer "B.Cu") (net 19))
 (segment (start 105.161101 110.66) (end 106.81 110.66) (width 0.5) (layer "B.Cu") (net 19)))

